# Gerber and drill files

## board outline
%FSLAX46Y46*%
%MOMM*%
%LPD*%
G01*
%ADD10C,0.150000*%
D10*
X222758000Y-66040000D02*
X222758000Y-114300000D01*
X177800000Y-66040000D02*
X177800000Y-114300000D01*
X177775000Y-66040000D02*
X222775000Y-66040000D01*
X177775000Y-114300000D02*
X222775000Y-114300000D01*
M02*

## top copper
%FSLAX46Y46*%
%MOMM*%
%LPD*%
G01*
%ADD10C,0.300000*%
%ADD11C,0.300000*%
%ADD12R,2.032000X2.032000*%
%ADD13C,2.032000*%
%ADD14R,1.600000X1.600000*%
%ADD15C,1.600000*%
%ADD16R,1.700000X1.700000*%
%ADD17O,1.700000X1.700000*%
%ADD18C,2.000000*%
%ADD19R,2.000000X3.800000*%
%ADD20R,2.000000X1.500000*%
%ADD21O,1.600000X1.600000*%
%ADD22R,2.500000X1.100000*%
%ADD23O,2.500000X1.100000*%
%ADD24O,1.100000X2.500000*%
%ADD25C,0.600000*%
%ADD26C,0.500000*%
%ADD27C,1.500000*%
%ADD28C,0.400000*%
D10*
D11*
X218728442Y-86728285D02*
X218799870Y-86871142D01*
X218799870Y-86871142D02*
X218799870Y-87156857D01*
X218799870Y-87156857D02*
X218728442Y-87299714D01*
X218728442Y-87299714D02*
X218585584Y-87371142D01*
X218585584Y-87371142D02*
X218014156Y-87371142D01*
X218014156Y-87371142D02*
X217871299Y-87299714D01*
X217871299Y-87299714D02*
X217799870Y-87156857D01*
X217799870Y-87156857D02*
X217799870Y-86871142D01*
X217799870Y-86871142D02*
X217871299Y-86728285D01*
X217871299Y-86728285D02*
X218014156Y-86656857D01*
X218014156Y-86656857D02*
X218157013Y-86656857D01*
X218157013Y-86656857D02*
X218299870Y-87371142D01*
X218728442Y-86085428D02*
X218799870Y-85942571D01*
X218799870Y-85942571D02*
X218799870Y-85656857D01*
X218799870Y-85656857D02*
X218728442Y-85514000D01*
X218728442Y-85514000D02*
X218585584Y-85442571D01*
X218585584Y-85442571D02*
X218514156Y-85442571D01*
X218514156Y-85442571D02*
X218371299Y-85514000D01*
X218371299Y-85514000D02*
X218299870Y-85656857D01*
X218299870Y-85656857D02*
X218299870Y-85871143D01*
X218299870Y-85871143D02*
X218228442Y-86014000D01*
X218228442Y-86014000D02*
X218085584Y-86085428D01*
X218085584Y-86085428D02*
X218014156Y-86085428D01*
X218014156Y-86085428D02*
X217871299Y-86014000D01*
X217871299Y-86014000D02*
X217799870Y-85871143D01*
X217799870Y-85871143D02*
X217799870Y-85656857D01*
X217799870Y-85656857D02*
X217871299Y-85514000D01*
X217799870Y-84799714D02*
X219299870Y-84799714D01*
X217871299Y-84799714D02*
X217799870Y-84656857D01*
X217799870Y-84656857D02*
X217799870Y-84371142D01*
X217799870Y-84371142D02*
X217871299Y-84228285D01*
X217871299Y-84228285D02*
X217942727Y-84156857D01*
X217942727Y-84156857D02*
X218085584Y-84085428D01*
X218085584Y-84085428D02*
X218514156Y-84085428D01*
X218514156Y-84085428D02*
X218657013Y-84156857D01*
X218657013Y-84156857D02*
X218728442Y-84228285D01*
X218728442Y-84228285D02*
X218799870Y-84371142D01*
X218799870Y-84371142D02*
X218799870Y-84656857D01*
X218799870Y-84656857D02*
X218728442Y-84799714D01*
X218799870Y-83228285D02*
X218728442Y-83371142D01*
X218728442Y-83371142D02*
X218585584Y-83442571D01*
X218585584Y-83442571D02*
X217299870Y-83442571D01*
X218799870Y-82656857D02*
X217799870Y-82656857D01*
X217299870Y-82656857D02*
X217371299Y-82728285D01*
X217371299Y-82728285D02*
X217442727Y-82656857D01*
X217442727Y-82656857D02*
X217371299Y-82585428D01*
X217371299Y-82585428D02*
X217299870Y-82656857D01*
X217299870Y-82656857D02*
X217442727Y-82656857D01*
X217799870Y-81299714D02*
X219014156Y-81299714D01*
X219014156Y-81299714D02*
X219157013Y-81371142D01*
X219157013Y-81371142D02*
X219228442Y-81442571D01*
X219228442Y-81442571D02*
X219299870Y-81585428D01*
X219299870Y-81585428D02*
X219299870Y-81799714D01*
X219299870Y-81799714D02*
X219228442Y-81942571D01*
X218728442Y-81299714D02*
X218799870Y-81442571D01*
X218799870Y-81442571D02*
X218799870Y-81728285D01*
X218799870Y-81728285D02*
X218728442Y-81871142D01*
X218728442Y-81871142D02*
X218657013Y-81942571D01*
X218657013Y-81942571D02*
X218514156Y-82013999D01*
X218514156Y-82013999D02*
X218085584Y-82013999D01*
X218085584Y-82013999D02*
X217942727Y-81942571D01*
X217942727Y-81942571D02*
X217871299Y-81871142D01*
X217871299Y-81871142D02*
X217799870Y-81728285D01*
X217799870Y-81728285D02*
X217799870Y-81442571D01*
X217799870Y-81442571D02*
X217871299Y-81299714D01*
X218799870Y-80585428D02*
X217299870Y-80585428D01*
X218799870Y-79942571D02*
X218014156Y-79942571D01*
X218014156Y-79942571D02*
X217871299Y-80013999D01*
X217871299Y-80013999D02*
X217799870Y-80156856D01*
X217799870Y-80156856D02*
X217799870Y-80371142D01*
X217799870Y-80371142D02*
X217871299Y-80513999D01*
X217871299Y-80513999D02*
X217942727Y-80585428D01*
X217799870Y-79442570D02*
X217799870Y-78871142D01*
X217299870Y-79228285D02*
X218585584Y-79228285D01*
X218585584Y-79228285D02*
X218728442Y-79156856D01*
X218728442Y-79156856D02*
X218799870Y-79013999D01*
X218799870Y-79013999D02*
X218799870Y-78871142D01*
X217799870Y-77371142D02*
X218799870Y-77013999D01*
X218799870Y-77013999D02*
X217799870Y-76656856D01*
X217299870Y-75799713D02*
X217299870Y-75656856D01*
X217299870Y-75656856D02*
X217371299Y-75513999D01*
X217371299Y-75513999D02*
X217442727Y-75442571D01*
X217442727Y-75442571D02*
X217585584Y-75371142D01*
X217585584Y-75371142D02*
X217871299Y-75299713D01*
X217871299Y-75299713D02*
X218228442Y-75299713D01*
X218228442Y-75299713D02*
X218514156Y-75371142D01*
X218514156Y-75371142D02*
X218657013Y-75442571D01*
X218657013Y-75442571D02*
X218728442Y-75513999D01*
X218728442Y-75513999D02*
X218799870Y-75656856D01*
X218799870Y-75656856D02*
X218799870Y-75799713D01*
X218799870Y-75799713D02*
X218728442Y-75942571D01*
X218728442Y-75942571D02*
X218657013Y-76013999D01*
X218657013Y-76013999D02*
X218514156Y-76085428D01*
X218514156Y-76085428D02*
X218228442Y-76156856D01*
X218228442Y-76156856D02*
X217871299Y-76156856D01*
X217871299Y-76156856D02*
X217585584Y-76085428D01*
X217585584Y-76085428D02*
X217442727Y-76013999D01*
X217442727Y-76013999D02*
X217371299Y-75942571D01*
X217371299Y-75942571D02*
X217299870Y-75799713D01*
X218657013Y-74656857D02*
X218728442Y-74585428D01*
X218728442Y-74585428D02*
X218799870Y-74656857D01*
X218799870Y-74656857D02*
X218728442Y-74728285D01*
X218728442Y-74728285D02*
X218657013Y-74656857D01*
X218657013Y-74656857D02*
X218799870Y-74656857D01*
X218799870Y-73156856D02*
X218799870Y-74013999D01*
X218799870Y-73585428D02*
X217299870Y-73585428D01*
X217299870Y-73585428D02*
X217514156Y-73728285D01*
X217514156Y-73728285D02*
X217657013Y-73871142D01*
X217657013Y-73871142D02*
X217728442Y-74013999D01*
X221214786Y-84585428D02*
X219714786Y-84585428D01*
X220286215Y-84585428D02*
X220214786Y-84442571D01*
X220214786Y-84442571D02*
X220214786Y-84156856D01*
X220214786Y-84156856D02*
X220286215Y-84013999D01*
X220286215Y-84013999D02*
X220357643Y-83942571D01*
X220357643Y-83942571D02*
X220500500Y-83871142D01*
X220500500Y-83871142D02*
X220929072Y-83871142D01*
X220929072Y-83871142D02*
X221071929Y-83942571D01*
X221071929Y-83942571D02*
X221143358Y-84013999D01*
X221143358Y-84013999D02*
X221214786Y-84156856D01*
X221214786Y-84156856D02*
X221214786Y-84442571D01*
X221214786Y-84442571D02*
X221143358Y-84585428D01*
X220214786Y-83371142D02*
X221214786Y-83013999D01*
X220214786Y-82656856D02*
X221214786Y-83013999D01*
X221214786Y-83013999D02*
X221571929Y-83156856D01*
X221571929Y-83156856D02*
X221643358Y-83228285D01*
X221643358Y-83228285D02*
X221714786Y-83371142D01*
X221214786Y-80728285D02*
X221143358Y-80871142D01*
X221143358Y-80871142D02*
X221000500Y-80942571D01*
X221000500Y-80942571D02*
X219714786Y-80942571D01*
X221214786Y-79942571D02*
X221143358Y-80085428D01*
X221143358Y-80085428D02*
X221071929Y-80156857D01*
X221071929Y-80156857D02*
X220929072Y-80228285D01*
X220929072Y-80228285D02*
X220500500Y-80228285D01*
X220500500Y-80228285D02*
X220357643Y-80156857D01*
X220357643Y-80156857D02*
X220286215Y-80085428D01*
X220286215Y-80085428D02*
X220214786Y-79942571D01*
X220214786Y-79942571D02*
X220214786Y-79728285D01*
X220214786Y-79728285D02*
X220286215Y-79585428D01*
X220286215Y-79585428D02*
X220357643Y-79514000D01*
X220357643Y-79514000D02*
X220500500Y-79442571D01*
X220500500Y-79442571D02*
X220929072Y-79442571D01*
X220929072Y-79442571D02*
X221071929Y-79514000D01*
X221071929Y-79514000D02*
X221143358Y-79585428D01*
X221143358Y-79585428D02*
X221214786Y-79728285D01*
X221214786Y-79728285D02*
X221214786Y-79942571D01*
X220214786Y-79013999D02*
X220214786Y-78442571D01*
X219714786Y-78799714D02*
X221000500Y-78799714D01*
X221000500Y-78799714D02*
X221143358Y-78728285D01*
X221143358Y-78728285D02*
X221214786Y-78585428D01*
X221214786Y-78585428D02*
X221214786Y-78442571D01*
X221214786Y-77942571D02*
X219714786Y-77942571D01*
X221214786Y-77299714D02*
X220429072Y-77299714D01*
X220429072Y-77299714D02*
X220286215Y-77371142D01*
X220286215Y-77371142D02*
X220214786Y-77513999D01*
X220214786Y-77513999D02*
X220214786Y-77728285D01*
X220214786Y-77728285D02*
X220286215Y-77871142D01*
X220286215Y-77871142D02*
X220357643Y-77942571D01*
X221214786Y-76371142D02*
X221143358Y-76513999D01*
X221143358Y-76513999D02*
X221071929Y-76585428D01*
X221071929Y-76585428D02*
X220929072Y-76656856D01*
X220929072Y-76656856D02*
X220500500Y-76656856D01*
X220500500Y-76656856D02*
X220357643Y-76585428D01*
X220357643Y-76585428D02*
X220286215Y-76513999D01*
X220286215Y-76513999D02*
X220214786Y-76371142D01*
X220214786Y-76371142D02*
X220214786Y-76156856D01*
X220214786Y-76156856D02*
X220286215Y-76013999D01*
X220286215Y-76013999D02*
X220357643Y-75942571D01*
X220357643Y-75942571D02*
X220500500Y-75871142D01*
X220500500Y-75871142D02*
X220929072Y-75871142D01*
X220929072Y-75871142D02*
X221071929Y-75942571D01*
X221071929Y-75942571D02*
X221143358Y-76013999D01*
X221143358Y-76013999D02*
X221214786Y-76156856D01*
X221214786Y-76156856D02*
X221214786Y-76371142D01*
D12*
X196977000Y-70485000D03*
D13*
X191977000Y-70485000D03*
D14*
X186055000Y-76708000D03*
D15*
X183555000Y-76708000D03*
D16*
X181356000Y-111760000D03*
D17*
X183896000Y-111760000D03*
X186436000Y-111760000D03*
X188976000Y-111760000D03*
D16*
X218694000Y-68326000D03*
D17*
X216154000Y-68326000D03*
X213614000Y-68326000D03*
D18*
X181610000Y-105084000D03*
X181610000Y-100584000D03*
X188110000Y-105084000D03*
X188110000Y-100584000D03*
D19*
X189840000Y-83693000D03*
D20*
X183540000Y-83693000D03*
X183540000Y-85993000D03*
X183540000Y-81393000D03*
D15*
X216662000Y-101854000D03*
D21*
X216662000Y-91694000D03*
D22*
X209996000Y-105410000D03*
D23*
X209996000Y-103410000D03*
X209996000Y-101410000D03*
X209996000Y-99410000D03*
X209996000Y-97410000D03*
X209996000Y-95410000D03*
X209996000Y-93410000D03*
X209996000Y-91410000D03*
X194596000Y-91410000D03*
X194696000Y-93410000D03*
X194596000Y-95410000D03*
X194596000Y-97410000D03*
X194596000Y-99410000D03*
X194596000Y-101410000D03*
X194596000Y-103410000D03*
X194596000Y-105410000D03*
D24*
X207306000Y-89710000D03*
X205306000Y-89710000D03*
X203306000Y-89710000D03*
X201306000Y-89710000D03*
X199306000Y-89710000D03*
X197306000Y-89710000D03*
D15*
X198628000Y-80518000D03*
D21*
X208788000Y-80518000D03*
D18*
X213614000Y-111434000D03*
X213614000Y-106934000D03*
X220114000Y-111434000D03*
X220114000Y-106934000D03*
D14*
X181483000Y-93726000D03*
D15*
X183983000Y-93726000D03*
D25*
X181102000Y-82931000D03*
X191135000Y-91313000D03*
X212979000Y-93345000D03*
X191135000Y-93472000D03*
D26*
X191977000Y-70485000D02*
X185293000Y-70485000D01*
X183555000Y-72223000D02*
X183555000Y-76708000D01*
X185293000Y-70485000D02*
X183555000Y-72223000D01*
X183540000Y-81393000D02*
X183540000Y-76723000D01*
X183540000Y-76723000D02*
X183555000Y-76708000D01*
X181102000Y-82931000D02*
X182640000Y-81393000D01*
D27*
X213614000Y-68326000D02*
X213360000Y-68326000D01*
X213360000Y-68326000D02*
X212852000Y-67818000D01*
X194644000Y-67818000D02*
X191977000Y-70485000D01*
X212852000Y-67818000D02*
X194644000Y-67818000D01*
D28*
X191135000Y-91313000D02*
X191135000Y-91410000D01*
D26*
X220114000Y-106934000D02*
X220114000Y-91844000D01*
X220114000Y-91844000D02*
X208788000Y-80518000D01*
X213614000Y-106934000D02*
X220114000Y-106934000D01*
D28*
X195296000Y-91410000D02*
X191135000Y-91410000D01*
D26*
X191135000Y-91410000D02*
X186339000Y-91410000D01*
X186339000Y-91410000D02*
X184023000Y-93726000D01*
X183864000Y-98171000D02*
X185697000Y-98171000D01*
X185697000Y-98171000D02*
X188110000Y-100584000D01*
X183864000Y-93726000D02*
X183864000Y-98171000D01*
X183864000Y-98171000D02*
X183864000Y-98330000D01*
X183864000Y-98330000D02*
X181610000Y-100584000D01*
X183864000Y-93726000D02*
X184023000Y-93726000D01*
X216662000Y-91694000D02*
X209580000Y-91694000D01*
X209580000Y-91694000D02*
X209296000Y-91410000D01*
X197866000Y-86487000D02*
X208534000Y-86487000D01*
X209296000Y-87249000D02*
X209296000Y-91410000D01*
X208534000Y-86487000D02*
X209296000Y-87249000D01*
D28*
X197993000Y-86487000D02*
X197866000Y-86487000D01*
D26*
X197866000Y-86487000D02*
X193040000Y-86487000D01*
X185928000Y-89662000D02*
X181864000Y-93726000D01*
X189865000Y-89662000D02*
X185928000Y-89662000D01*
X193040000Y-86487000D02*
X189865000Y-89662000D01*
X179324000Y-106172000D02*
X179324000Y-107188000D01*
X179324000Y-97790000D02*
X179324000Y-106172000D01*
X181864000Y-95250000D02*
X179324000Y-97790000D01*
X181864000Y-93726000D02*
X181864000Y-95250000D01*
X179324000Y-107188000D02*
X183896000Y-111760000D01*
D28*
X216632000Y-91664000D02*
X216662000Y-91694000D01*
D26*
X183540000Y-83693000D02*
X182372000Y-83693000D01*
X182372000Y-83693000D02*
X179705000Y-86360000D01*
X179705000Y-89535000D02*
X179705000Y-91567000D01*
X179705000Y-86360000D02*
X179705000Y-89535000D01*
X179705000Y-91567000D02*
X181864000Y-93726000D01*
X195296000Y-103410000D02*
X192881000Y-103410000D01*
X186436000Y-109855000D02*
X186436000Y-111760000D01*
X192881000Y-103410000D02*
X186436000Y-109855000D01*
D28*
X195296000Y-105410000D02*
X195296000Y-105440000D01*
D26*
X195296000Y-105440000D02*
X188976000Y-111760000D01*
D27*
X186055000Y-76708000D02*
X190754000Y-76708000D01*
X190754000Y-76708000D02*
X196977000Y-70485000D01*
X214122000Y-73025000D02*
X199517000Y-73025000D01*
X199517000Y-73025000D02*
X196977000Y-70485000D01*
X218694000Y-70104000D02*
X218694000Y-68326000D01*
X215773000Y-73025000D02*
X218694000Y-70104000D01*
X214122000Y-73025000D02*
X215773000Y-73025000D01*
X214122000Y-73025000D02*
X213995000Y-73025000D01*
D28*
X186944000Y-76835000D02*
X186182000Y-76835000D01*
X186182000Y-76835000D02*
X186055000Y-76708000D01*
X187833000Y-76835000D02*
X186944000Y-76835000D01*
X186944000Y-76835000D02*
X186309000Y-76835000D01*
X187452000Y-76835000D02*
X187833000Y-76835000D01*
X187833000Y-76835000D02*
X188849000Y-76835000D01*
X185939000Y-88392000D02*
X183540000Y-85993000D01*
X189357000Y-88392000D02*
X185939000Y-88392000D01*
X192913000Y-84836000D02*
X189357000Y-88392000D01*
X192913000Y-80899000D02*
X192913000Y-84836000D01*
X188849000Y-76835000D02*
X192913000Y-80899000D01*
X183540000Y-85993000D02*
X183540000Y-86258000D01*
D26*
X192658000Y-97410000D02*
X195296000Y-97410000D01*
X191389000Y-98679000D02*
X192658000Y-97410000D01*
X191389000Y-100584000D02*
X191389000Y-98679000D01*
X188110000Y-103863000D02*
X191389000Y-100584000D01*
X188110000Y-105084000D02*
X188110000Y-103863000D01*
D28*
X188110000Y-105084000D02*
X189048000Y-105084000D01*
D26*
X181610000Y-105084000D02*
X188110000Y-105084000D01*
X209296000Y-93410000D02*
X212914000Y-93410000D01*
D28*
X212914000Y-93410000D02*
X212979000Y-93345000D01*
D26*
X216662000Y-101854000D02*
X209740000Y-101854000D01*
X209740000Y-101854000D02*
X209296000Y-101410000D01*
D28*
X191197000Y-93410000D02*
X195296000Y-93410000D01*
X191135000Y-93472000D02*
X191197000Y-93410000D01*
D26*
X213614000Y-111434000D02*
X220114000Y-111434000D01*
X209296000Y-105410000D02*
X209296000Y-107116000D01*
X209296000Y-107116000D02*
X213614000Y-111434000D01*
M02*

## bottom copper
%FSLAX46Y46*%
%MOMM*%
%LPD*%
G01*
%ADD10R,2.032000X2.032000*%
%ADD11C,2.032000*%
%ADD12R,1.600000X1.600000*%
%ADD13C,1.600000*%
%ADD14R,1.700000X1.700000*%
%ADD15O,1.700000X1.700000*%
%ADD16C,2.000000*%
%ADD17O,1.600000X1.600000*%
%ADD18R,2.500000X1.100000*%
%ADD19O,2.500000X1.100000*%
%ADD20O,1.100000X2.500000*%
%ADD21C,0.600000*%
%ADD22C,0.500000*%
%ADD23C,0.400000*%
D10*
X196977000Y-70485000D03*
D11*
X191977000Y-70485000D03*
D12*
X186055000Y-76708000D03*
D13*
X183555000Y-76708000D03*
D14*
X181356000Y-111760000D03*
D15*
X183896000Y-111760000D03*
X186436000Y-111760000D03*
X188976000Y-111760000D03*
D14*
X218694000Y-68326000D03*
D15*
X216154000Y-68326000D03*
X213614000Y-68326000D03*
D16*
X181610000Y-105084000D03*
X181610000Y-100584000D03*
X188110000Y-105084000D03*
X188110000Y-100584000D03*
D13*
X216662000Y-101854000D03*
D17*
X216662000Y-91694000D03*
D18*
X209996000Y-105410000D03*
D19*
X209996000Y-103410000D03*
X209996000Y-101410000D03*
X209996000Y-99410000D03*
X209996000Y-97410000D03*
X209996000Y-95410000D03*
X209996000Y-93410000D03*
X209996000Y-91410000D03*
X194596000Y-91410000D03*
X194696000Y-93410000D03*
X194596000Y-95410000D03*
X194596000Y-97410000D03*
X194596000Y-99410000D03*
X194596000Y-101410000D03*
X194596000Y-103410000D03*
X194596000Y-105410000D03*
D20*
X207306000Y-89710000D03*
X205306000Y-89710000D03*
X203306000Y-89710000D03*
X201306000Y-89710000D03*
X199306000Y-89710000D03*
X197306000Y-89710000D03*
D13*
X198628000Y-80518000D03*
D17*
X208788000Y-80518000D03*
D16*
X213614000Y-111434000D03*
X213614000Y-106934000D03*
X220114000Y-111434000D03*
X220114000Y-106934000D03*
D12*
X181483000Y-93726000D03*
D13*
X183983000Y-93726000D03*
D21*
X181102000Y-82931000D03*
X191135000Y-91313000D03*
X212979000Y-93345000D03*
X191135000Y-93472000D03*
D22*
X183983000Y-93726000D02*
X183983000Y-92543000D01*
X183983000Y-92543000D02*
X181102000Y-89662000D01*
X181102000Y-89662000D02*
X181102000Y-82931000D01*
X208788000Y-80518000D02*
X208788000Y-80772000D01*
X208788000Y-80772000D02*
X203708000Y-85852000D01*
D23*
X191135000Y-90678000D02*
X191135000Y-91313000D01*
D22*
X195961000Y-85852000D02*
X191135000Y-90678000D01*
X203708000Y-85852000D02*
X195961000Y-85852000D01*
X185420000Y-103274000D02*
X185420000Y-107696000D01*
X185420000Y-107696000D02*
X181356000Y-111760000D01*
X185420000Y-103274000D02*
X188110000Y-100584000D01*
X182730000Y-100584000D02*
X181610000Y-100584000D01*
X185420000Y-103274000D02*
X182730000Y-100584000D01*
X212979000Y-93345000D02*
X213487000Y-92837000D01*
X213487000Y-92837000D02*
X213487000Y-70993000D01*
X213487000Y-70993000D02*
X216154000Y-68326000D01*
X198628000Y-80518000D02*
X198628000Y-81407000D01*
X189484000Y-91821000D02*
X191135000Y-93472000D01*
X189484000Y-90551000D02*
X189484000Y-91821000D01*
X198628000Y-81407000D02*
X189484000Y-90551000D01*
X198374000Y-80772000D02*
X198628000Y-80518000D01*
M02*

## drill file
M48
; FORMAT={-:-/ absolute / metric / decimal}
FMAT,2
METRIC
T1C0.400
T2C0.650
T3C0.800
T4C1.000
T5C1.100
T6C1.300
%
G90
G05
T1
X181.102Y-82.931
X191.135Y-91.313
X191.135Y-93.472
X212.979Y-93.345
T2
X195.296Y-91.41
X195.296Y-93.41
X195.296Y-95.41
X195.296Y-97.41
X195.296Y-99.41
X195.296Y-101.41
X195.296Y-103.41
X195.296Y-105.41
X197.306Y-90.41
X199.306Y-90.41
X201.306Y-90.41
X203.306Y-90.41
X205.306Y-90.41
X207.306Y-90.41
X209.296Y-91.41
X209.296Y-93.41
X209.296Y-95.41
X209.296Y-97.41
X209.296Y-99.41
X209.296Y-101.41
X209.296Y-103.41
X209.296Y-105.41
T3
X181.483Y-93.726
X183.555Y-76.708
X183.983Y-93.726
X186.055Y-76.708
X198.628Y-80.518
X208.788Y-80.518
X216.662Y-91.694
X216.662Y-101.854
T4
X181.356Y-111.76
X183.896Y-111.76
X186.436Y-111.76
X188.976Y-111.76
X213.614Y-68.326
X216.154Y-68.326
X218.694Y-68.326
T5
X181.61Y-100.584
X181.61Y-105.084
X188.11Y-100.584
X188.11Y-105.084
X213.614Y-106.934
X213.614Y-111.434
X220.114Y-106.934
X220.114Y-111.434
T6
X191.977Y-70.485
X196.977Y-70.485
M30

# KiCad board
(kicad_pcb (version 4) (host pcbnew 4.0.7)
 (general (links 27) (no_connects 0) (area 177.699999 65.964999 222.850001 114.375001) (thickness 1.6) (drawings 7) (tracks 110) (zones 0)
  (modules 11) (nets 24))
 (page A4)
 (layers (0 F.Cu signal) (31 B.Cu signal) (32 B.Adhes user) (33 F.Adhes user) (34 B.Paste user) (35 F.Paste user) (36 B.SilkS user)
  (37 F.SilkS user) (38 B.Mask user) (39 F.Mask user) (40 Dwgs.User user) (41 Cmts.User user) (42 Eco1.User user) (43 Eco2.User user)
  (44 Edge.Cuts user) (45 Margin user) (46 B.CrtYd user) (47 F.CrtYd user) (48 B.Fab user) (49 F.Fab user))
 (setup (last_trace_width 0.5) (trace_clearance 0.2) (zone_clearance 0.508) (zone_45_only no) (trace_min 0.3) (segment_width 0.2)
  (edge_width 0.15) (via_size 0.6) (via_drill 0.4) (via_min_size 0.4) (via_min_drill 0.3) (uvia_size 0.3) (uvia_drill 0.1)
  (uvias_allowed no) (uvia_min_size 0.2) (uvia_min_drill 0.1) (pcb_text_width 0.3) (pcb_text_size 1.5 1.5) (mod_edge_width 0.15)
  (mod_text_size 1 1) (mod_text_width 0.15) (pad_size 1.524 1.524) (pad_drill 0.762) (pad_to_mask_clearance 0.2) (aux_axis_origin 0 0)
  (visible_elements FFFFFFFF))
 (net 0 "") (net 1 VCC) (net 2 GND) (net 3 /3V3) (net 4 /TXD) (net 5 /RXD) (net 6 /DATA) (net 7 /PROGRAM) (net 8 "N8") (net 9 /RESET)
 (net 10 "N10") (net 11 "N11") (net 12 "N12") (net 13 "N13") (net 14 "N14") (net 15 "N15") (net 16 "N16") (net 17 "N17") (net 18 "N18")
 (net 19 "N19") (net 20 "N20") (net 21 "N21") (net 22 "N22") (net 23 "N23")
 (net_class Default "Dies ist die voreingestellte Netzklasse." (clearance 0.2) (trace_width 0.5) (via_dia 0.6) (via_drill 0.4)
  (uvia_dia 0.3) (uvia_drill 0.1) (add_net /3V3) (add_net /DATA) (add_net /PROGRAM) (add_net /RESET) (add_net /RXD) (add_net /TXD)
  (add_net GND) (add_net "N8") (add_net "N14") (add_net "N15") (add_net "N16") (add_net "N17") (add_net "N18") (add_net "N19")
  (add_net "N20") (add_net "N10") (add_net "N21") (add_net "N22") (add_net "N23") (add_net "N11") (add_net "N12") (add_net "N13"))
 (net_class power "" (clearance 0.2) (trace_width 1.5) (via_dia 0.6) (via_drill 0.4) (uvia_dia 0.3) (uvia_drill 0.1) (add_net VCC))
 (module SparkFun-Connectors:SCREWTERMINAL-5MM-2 (layer F.Cu) (at 196.977 70.485 180)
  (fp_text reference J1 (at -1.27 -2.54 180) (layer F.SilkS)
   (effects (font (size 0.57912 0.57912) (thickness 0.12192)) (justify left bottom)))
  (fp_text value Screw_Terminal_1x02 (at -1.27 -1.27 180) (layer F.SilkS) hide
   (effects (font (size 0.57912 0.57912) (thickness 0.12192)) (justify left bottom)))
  (pad 1 thru_hole rect (at 0 0 180) (size 2.032 2.032) (drill 1.3) (layers *.Cu *.Mask) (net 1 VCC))
  (pad 2 thru_hole circle (at 5 0 180) (size 2.032 2.032) (drill 1.3) (layers *.Cu *.Mask) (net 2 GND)))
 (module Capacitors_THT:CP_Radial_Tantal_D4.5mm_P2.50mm (layer F.Cu) (at 186.055 76.708 180)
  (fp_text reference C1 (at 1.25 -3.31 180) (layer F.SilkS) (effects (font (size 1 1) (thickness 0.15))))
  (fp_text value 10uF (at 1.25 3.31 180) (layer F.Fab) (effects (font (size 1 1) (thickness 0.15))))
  (pad 1 thru_hole rect (at 0 0 180) (size 1.6 1.6) (drill 0.8) (layers *.Cu *.Mask) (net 1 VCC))
  (pad 2 thru_hole circle (at 2.5 0 180) (size 1.6 1.6) (drill 0.8) (layers *.Cu *.Mask) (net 2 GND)))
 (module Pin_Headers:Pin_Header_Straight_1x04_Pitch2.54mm (layer F.Cu) (at 181.356 111.76 90)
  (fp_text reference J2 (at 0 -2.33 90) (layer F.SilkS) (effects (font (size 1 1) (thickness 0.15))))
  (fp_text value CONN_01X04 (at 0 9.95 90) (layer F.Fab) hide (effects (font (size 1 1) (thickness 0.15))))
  (pad 1 thru_hole rect (at 0 0 90) (size 1.7 1.7) (drill 1) (layers *.Cu *.Mask) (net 2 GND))
  (pad 2 thru_hole oval (at 0 2.54 90) (size 1.7 1.7) (drill 1) (layers *.Cu *.Mask) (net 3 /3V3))
  (pad 3 thru_hole oval (at 0 5.08 90) (size 1.7 1.7) (drill 1) (layers *.Cu *.Mask) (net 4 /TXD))
  (pad 4 thru_hole oval (at 0 7.62 90) (size 1.7 1.7) (drill 1) (layers *.Cu *.Mask) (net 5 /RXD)))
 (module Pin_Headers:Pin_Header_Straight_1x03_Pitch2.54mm (layer F.Cu) (at 218.694 68.326 270)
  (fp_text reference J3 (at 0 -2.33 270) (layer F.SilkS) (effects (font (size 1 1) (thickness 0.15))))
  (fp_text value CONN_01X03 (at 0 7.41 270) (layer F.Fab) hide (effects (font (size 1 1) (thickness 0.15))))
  (pad 1 thru_hole rect (at 0 0 270) (size 1.7 1.7) (drill 1) (layers *.Cu *.Mask) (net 1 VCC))
  (pad 2 thru_hole oval (at 0 2.54 270) (size 1.7 1.7) (drill 1) (layers *.Cu *.Mask) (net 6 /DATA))
  (pad 3 thru_hole oval (at 0 5.08 270) (size 1.7 1.7) (drill 1) (layers *.Cu *.Mask) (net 2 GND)))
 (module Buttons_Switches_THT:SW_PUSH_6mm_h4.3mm (layer F.Cu) (at 181.61 100.584)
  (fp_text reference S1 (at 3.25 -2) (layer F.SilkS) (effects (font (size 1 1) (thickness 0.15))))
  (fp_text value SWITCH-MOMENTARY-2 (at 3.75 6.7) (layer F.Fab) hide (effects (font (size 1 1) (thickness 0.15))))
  (pad 2 thru_hole circle (at 0 4.5 90) (size 2 2) (drill 1.1) (layers *.Cu *.Mask) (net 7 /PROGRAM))
  (pad 1 thru_hole circle (at 0 0 90) (size 2 2) (drill 1.1) (layers *.Cu *.Mask) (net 2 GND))
  (pad 2 thru_hole circle (at 6.5 4.5 90) (size 2 2) (drill 1.1) (layers *.Cu *.Mask) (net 7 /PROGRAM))
  (pad 1 thru_hole circle (at 6.5 0 90) (size 2 2) (drill 1.1) (layers *.Cu *.Mask) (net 2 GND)))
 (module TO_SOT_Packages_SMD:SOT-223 (layer F.Cu) (at 186.69 83.693)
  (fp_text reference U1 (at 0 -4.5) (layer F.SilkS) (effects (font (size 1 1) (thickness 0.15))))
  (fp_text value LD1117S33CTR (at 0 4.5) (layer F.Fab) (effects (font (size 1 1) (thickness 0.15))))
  (pad 4 smd rect (at 3.15 0) (size 2 3.8) (layers F.Cu F.Paste F.Mask))
  (pad 2 smd rect (at -3.15 0) (size 2 1.5) (layers F.Cu F.Paste F.Mask) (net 3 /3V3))
  (pad 3 smd rect (at -3.15 2.3) (size 2 1.5) (layers F.Cu F.Paste F.Mask) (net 1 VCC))
  (pad 1 smd rect (at -3.15 -2.3) (size 2 1.5) (layers F.Cu F.Paste F.Mask) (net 2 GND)))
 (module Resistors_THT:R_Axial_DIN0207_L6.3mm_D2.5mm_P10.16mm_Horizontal (layer F.Cu) (at 216.662 101.854 90)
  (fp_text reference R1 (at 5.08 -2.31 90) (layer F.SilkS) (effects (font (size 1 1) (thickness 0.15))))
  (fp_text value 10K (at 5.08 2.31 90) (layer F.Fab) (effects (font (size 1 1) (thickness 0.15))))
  (pad 1 thru_hole circle (at 0 0 90) (size 1.6 1.6) (drill 0.8) (layers *.Cu *.Mask) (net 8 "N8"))
  (pad 2 thru_hole oval (at 10.16 0 90) (size 1.6 1.6) (drill 0.8) (layers *.Cu *.Mask) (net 3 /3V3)))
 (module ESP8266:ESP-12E (layer F.Cu) (at 209.296 105.41 180)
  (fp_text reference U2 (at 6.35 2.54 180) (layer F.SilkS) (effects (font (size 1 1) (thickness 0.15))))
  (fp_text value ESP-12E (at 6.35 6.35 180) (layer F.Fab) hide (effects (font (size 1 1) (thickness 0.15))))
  (pad 1 thru_hole rect (at 0 0 180) (size 2.5 1.1) (drill 0.65 (offset -0.7 0)) (layers *.Cu *.Mask F.SilkS) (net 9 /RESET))
  (pad 2 thru_hole oval (at 0 2 180) (size 2.5 1.1) (drill 0.65 (offset -0.7 0)) (layers *.Cu *.Mask F.SilkS) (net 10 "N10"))
  (pad 3 thru_hole oval (at 0 4 180) (size 2.5 1.1) (drill 0.65 (offset -0.7 0)) (layers *.Cu *.Mask F.SilkS) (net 8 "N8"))
  (pad 4 thru_hole oval (at 0 6 180) (size 2.5 1.1) (drill 0.65 (offset -0.7 0)) (layers *.Cu *.Mask F.SilkS) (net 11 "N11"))
  (pad 5 thru_hole oval (at 0 8 180) (size 2.5 1.1) (drill 0.65 (offset -0.7 0)) (layers *.Cu *.Mask F.SilkS) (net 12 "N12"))
  (pad 6 thru_hole oval (at 0 10 180) (size 2.5 1.1) (drill 0.65 (offset -0.7 0)) (layers *.Cu *.Mask F.SilkS) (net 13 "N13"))
  (pad 7 thru_hole oval (at 0 12 180) (size 2.5 1.1) (drill 0.65 (offset -0.7 0)) (layers *.Cu *.Mask F.SilkS) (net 6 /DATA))
  (pad 8 thru_hole oval (at 0 14 180) (size 2.5 1.1) (drill 0.65 (offset -0.7 0)) (layers *.Cu *.Mask F.SilkS) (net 3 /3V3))
  (pad 9 thru_hole oval (at 14 14 180) (size 2.5 1.1) (drill 0.65 (offset 0.7 0)) (layers *.Cu *.Mask F.SilkS) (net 2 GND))
  (pad 10 thru_hole oval (at 14 12 180) (size 2.5 1.1) (drill 0.65 (offset 0.6 0)) (layers *.Cu *.Mask F.SilkS) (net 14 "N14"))
  (pad 11 thru_hole oval (at 14 10 180) (size 2.5 1.1) (drill 0.65 (offset 0.7 0)) (layers *.Cu *.Mask F.SilkS) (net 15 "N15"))
  (pad 12 thru_hole oval (at 14 8 180) (size 2.5 1.1) (drill 0.65 (offset 0.7 0)) (layers *.Cu *.Mask F.SilkS) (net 7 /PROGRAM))
  (pad 13 thru_hole oval (at 14 6 180) (size 2.5 1.1) (drill 0.65 (offset 0.7 0)) (layers *.Cu *.Mask F.SilkS) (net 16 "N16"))
  (pad 14 thru_hole oval (at 14 4 180) (size 2.5 1.1) (drill 0.65 (offset 0.7 0)) (layers *.Cu *.Mask F.SilkS) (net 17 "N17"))
  (pad 15 thru_hole oval (at 14 2 180) (size 2.5 1.1) (drill 0.65 (offset 0.7 0)) (layers *.Cu *.Mask F.SilkS) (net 4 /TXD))
  (pad 16 thru_hole oval (at 14 0 180) (size 2.5 1.1) (drill 0.65 (offset 0.7 0)) (layers *.Cu *.Mask F.SilkS) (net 5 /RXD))
  (pad 17 thru_hole oval (at 1.99 15 270) (size 2.5 1.1) (drill 0.65 (offset -0.7 0)) (layers *.Cu *.Mask F.SilkS) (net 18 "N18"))
  (pad 18 thru_hole oval (at 3.99 15 270) (size 2.5 1.1) (drill 0.65 (offset -0.7 0)) (layers *.Cu *.Mask F.SilkS) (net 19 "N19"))
  (pad 19 thru_hole oval (at 5.99 15 270) (size 2.5 1.1) (drill 0.65 (offset -0.7 0)) (layers *.Cu *.Mask F.SilkS) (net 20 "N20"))
  (pad 20 thru_hole oval (at 7.99 15 270) (size 2.5 1.1) (drill 0.65 (offset -0.7 0)) (layers *.Cu *.Mask F.SilkS) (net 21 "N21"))
  (pad 21 thru_hole oval (at 9.99 15 270) (size 2.5 1.1) (drill 0.65 (offset -0.7 0)) (layers *.Cu *.Mask F.SilkS) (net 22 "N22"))
  (pad 22 thru_hole oval (at 11.99 15 270) (size 2.5 1.1) (drill 0.65 (offset -0.7 0)) (layers *.Cu *.Mask F.SilkS) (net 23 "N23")))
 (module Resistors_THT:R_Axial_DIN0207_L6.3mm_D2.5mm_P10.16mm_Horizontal (layer F.Cu) (at 198.628 80.518)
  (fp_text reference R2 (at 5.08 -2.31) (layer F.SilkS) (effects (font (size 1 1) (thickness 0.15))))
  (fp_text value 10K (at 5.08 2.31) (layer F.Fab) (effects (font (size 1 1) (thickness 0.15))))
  (pad 1 thru_hole circle (at 0 0) (size 1.6 1.6) (drill 0.8) (layers *.Cu *.Mask) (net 14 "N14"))
  (pad 2 thru_hole oval (at 10.16 0) (size 1.6 1.6) (drill 0.8) (layers *.Cu *.Mask) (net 2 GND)))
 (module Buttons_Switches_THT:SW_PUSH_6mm (layer F.Cu) (at 213.614 106.934)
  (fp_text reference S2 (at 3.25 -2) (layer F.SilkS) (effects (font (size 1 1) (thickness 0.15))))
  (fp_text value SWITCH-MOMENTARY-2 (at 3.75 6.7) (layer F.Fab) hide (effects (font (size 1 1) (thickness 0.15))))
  (pad 2 thru_hole circle (at 0 4.5 90) (size 2 2) (drill 1.1) (layers *.Cu *.Mask) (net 9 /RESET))
  (pad 1 thru_hole circle (at 0 0 90) (size 2 2) (drill 1.1) (layers *.Cu *.Mask) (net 2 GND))
  (pad 2 thru_hole circle (at 6.5 4.5 90) (size 2 2) (drill 1.1) (layers *.Cu *.Mask) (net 9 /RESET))
  (pad 1 thru_hole circle (at 6.5 0 90) (size 2 2) (drill 1.1) (layers *.Cu *.Mask) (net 2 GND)))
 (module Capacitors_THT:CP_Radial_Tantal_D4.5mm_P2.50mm (layer F.Cu) (at 181.483 93.726)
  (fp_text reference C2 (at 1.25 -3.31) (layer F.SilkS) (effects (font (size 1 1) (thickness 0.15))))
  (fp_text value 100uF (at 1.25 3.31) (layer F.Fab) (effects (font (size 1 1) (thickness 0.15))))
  (pad 1 thru_hole rect (at 0 0) (size 1.6 1.6) (drill 0.8) (layers *.Cu *.Mask) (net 3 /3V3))
  (pad 2 thru_hole circle (at 2.5 0) (size 1.6 1.6) (drill 0.8) (layers *.Cu *.Mask) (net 2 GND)))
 (gr_line (start 222.758 66.04) (end 222.758 114.3) (angle 90) (layer Edge.Cuts) (width 0.15))
 (gr_line (start 177.8 66.04) (end 177.8 114.3) (angle 90) (layer Edge.Cuts) (width 0.15))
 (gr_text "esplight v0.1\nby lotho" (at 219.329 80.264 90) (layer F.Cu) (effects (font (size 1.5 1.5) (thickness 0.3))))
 (gr_line (start 177.775 66.04) (end 222.775 66.04) (angle 90) (layer Edge.Cuts) (width 0.15))
 (gr_line (start 177.775 114.3) (end 222.775 114.3) (angle 90) (layer Edge.Cuts) (width 0.15))
 (segment (start 191.977 70.485) (end 185.293 70.485) (width 0.5) (layer F.Cu) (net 2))
 (segment (start 183.555 72.223) (end 183.555 76.708) (width 0.5) (layer F.Cu) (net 2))
 (segment (start 185.293 70.485) (end 183.555 72.223) (width 0.5) (layer F.Cu) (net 2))
 (segment (start 183.54 81.393) (end 183.54 76.723) (width 0.5) (layer F.Cu) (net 2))
 (segment (start 183.54 76.723) (end 183.555 76.708) (width 0.5) (layer F.Cu) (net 2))
 (segment (start 183.983 93.726) (end 183.983 92.543) (width 0.5) (layer B.Cu) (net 2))
 (segment (start 183.983 92.543) (end 181.102 89.662) (width 0.5) (layer B.Cu) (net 2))
 (segment (start 181.102 89.662) (end 181.102 82.931) (width 0.5) (layer B.Cu) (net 2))
 (via (at 181.102 82.931) (size 0.6) (drill 0.4) (layers F.Cu B.Cu) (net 2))
 (segment (start 181.102 82.931) (end 182.64 81.393) (width 0.5) (layer F.Cu) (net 2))
 (segment (start 213.614 68.326) (end 213.36 68.326) (width 1.5) (layer F.Cu) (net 2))
 (segment (start 213.36 68.326) (end 212.852 67.818) (width 1.5) (layer F.Cu) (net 2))
 (segment (start 194.644 67.818) (end 191.977 70.485) (width 1.5) (layer F.Cu) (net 2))
 (segment (start 212.852 67.818) (end 194.644 67.818) (width 1.5) (layer F.Cu) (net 2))
 (segment (start 208.788 80.518) (end 208.788 80.772) (width 0.5) (layer B.Cu) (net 2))
 (segment (start 208.788 80.772) (end 203.708 85.852) (width 0.5) (layer B.Cu) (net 2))
 (segment (start 191.135 91.313) (end 191.135 91.41) (width 0.4) (layer F.Cu) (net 2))
 (via (at 191.135 91.313) (size 0.6) (drill 0.4) (layers F.Cu B.Cu) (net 2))
 (segment (start 191.135 90.678) (end 191.135 91.313) (width 0.4) (layer B.Cu) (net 2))
 (segment (start 195.961 85.852) (end 191.135 90.678) (width 0.5) (layer B.Cu) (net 2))
 (segment (start 203.708 85.852) (end 195.961 85.852) (width 0.5) (layer B.Cu) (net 2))
 (segment (start 220.114 106.934) (end 220.114 91.844) (width 0.5) (layer F.Cu) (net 2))
 (segment (start 220.114 91.844) (end 208.788 80.518) (width 0.5) (layer F.Cu) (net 2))
 (segment (start 213.614 106.934) (end 220.114 106.934) (width 0.5) (layer F.Cu) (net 2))
 (segment (start 195.296 91.41) (end 191.135 91.41) (width 0.4) (layer F.Cu) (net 2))
 (segment (start 191.135 91.41) (end 186.339 91.41) (width 0.5) (layer F.Cu) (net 2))
 (segment (start 186.339 91.41) (end 184.023 93.726) (width 0.5) (layer F.Cu) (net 2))
 (segment (start 185.42 103.274) (end 185.42 107.696) (width 0.5) (layer B.Cu) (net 2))
 (segment (start 185.42 107.696) (end 181.356 111.76) (width 0.5) (layer B.Cu) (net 2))
 (segment (start 185.42 103.274) (end 188.11 100.584) (width 0.5) (layer B.Cu) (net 2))
 (segment (start 182.73 100.584) (end 181.61 100.584) (width 0.5) (layer B.Cu) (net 2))
 (segment (start 185.42 103.274) (end 182.73 100.584) (width 0.5) (layer B.Cu) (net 2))
 (segment (start 183.864 98.171) (end 185.697 98.171) (width 0.5) (layer F.Cu) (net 2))
 (segment (start 185.697 98.171) (end 188.11 100.584) (width 0.5) (layer F.Cu) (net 2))
 (segment (start 183.864 93.726) (end 183.864 98.171) (width 0.5) (layer F.Cu) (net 2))
 (segment (start 183.864 98.171) (end 183.864 98.33) (width 0.5) (layer F.Cu) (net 2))
 (segment (start 183.864 98.33) (end 181.61 100.584) (width 0.5) (layer F.Cu) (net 2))
 (segment (start 183.864 93.726) (end 184.023 93.726) (width 0.5) (layer F.Cu) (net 2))
 (segment (start 216.662 91.694) (end 209.58 91.694) (width 0.5) (layer F.Cu) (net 3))
 (segment (start 209.58 91.694) (end 209.296 91.41) (width 0.5) (layer F.Cu) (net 3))
 (segment (start 197.866 86.487) (end 208.534 86.487) (width 0.5) (layer F.Cu) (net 3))
 (segment (start 209.296 87.249) (end 209.296 91.41) (width 0.5) (layer F.Cu) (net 3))
 (segment (start 208.534 86.487) (end 209.296 87.249) (width 0.5) (layer F.Cu) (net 3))
 (segment (start 197.993 86.487) (end 197.866 86.487) (width 0.4) (layer F.Cu) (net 3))
 (segment (start 197.866 86.487) (end 193.04 86.487) (width 0.5) (layer F.Cu) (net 3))
 (segment (start 185.928 89.662) (end 181.864 93.726) (width 0.5) (layer F.Cu) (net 3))
 (segment (start 189.865 89.662) (end 185.928 89.662) (width 0.5) (layer F.Cu) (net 3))
 (segment (start 193.04 86.487) (end 189.865 89.662) (width 0.5) (layer F.Cu) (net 3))
 (segment (start 179.324 106.172) (end 179.324 107.188) (width 0.5) (layer F.Cu) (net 3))
 (segment (start 179.324 97.79) (end 179.324 106.172) (width 0.5) (layer F.Cu) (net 3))
 (segment (start 181.864 95.25) (end 179.324 97.79) (width 0.5) (layer F.Cu) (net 3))
 (segment (start 181.864 93.726) (end 181.864 95.25) (width 0.5) (layer F.Cu) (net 3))
 (segment (start 179.324 107.188) (end 183.896 111.76) (width 0.5) (layer F.Cu) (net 3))
 (segment (start 216.632 91.664) (end 216.662 91.694) (width 0.4) (layer F.Cu) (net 3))
 (segment (start 183.54 83.693) (end 182.372 83.693) (width 0.5) (layer F.Cu) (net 3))
 (segment (start 182.372 83.693) (end 179.705 86.36) (width 0.5) (layer F.Cu) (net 3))
 (segment (start 179.705 89.535) (end 179.705 91.567) (width 0.5) (layer F.Cu) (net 3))
 (segment (start 179.705 86.36) (end 179.705 89.535) (width 0.5) (layer F.Cu) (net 3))
 (segment (start 179.705 91.567) (end 181.864 93.726) (width 0.5) (layer F.Cu) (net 3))
 (segment (start 195.296 103.41) (end 192.881 103.41) (width 0.5) (layer F.Cu) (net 4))
 (segment (start 186.436 109.855) (end 186.436 111.76) (width 0.5) (layer F.Cu) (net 4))
 (segment (start 192.881 103.41) (end 186.436 109.855) (width 0.5) (layer F.Cu) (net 4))
 (segment (start 195.296 105.41) (end 195.296 105.44) (width 0.4) (layer F.Cu) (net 5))
 (segment (start 195.296 105.44) (end 188.976 111.76) (width 0.5) (layer F.Cu) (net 5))
 (segment (start 186.055 76.708) (end 190.754 76.708) (width 1.5) (layer F.Cu) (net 1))
 (segment (start 190.754 76.708) (end 196.977 70.485) (width 1.5) (layer F.Cu) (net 1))
 (segment (start 214.122 73.025) (end 199.517 73.025) (width 1.5) (layer F.Cu) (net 1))
 (segment (start 199.517 73.025) (end 196.977 70.485) (width 1.5) (layer F.Cu) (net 1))
 (segment (start 218.694 70.104) (end 218.694 68.326) (width 1.5) (layer F.Cu) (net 1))
 (segment (start 215.773 73.025) (end 218.694 70.104) (width 1.5) (layer F.Cu) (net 1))
 (segment (start 214.122 73.025) (end 215.773 73.025) (width 1.5) (layer F.Cu) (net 1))
 (segment (start 214.122 73.025) (end 213.995 73.025) (width 1.5) (layer F.Cu) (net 1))
 (segment (start 186.944 76.835) (end 186.182 76.835) (width 0.4) (layer F.Cu) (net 1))
 (segment (start 186.182 76.835) (end 186.055 76.708) (width 0.4) (layer F.Cu) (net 1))
 (segment (start 187.833 76.835) (end 186.944 76.835) (width 0.4) (layer F.Cu) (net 1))
 (segment (start 186.944 76.835) (end 186.309 76.835) (width 0.4) (layer F.Cu) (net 1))
 (segment (start 187.452 76.835) (end 187.833 76.835) (width 0.4) (layer F.Cu) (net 1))
 (segment (start 187.833 76.835) (end 188.849 76.835) (width 0.4) (layer F.Cu) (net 1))
 (segment (start 185.939 88.392) (end 183.54 85.993) (width 0.4) (layer F.Cu) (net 1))
 (segment (start 189.357 88.392) (end 185.939 88.392) (width 0.4) (layer F.Cu) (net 1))
 (segment (start 192.913 84.836) (end 189.357 88.392) (width 0.4) (layer F.Cu) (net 1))
 (segment (start 192.913 80.899) (end 192.913 84.836) (width 0.4) (layer F.Cu) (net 1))
 (segment (start 188.849 76.835) (end 192.913 80.899) (width 0.4) (layer F.Cu) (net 1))
 (segment (start 183.54 85.993) (end 183.54 86.258) (width 0.4) (layer F.Cu) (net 1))
 (segment (start 192.658 97.41) (end 195.296 97.41) (width 0.5) (layer F.Cu) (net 7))
 (segment (start 191.389 98.679) (end 192.658 97.41) (width 0.5) (layer F.Cu) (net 7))
 (segment (start 191.389 100.584) (end 191.389 98.679) (width 0.5) (layer F.Cu) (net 7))
 (segment (start 188.11 103.863) (end 191.389 100.584) (width 0.5) (layer F.Cu) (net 7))
 (segment (start 188.11 105.084) (end 188.11 103.863) (width 0.5) (layer F.Cu) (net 7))
 (segment (start 188.11 105.084) (end 189.048 105.084) (width 0.4) (layer F.Cu) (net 7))
 (segment (start 181.61 105.084) (end 188.11 105.084) (width 0.5) (layer F.Cu) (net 7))
 (segment (start 209.296 93.41) (end 212.914 93.41) (width 0.5) (layer F.Cu) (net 6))
 (segment (start 212.914 93.41) (end 212.979 93.345) (width 0.4) (layer F.Cu) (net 6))
 (via (at 212.979 93.345) (size 0.6) (drill 0.4) (layers F.Cu B.Cu) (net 6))
 (segment (start 212.979 93.345) (end 213.487 92.837) (width 0.5) (layer B.Cu) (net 6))
 (segment (start 213.487 92.837) (end 213.487 70.993) (width 0.5) (layer B.Cu) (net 6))
 (segment (start 213.487 70.993) (end 216.154 68.326) (width 0.5) (layer B.Cu) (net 6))
 (segment (start 216.662 101.854) (end 209.74 101.854) (width 0.5) (layer F.Cu) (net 8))
 (segment (start 209.74 101.854) (end 209.296 101.41) (width 0.5) (layer F.Cu) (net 8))
 (segment (start 198.628 80.518) (end 198.628 81.407) (width 0.5) (layer B.Cu) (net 14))
 (segment (start 191.197 93.41) (end 195.296 93.41) (width 0.4) (layer F.Cu) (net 14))
 (segment (start 191.135 93.472) (end 191.197 93.41) (width 0.4) (layer F.Cu) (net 14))
 (via (at 191.135 93.472) (size 0.6) (drill 0.4) (layers F.Cu B.Cu) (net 14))
 (segment (start 189.484 91.821) (end 191.135 93.472) (width 0.5) (layer B.Cu) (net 14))
 (segment (start 189.484 90.551) (end 189.484 91.821) (width 0.5) (layer B.Cu) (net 14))
 (segment (start 198.628 81.407) (end 189.484 90.551) (width 0.5) (layer B.Cu) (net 14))
 (segment (start 198.374 80.772) (end 198.628 80.518) (width 0.5) (layer B.Cu) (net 14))
 (segment (start 213.614 111.434) (end 220.114 111.434) (width 0.5) (layer F.Cu) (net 9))
 (segment (start 209.296 105.41) (end 209.296 107.116) (width 0.5) (layer F.Cu) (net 9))
 (segment (start 209.296 107.116) (end 213.614 111.434) (width 0.5) (layer F.Cu) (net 9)))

